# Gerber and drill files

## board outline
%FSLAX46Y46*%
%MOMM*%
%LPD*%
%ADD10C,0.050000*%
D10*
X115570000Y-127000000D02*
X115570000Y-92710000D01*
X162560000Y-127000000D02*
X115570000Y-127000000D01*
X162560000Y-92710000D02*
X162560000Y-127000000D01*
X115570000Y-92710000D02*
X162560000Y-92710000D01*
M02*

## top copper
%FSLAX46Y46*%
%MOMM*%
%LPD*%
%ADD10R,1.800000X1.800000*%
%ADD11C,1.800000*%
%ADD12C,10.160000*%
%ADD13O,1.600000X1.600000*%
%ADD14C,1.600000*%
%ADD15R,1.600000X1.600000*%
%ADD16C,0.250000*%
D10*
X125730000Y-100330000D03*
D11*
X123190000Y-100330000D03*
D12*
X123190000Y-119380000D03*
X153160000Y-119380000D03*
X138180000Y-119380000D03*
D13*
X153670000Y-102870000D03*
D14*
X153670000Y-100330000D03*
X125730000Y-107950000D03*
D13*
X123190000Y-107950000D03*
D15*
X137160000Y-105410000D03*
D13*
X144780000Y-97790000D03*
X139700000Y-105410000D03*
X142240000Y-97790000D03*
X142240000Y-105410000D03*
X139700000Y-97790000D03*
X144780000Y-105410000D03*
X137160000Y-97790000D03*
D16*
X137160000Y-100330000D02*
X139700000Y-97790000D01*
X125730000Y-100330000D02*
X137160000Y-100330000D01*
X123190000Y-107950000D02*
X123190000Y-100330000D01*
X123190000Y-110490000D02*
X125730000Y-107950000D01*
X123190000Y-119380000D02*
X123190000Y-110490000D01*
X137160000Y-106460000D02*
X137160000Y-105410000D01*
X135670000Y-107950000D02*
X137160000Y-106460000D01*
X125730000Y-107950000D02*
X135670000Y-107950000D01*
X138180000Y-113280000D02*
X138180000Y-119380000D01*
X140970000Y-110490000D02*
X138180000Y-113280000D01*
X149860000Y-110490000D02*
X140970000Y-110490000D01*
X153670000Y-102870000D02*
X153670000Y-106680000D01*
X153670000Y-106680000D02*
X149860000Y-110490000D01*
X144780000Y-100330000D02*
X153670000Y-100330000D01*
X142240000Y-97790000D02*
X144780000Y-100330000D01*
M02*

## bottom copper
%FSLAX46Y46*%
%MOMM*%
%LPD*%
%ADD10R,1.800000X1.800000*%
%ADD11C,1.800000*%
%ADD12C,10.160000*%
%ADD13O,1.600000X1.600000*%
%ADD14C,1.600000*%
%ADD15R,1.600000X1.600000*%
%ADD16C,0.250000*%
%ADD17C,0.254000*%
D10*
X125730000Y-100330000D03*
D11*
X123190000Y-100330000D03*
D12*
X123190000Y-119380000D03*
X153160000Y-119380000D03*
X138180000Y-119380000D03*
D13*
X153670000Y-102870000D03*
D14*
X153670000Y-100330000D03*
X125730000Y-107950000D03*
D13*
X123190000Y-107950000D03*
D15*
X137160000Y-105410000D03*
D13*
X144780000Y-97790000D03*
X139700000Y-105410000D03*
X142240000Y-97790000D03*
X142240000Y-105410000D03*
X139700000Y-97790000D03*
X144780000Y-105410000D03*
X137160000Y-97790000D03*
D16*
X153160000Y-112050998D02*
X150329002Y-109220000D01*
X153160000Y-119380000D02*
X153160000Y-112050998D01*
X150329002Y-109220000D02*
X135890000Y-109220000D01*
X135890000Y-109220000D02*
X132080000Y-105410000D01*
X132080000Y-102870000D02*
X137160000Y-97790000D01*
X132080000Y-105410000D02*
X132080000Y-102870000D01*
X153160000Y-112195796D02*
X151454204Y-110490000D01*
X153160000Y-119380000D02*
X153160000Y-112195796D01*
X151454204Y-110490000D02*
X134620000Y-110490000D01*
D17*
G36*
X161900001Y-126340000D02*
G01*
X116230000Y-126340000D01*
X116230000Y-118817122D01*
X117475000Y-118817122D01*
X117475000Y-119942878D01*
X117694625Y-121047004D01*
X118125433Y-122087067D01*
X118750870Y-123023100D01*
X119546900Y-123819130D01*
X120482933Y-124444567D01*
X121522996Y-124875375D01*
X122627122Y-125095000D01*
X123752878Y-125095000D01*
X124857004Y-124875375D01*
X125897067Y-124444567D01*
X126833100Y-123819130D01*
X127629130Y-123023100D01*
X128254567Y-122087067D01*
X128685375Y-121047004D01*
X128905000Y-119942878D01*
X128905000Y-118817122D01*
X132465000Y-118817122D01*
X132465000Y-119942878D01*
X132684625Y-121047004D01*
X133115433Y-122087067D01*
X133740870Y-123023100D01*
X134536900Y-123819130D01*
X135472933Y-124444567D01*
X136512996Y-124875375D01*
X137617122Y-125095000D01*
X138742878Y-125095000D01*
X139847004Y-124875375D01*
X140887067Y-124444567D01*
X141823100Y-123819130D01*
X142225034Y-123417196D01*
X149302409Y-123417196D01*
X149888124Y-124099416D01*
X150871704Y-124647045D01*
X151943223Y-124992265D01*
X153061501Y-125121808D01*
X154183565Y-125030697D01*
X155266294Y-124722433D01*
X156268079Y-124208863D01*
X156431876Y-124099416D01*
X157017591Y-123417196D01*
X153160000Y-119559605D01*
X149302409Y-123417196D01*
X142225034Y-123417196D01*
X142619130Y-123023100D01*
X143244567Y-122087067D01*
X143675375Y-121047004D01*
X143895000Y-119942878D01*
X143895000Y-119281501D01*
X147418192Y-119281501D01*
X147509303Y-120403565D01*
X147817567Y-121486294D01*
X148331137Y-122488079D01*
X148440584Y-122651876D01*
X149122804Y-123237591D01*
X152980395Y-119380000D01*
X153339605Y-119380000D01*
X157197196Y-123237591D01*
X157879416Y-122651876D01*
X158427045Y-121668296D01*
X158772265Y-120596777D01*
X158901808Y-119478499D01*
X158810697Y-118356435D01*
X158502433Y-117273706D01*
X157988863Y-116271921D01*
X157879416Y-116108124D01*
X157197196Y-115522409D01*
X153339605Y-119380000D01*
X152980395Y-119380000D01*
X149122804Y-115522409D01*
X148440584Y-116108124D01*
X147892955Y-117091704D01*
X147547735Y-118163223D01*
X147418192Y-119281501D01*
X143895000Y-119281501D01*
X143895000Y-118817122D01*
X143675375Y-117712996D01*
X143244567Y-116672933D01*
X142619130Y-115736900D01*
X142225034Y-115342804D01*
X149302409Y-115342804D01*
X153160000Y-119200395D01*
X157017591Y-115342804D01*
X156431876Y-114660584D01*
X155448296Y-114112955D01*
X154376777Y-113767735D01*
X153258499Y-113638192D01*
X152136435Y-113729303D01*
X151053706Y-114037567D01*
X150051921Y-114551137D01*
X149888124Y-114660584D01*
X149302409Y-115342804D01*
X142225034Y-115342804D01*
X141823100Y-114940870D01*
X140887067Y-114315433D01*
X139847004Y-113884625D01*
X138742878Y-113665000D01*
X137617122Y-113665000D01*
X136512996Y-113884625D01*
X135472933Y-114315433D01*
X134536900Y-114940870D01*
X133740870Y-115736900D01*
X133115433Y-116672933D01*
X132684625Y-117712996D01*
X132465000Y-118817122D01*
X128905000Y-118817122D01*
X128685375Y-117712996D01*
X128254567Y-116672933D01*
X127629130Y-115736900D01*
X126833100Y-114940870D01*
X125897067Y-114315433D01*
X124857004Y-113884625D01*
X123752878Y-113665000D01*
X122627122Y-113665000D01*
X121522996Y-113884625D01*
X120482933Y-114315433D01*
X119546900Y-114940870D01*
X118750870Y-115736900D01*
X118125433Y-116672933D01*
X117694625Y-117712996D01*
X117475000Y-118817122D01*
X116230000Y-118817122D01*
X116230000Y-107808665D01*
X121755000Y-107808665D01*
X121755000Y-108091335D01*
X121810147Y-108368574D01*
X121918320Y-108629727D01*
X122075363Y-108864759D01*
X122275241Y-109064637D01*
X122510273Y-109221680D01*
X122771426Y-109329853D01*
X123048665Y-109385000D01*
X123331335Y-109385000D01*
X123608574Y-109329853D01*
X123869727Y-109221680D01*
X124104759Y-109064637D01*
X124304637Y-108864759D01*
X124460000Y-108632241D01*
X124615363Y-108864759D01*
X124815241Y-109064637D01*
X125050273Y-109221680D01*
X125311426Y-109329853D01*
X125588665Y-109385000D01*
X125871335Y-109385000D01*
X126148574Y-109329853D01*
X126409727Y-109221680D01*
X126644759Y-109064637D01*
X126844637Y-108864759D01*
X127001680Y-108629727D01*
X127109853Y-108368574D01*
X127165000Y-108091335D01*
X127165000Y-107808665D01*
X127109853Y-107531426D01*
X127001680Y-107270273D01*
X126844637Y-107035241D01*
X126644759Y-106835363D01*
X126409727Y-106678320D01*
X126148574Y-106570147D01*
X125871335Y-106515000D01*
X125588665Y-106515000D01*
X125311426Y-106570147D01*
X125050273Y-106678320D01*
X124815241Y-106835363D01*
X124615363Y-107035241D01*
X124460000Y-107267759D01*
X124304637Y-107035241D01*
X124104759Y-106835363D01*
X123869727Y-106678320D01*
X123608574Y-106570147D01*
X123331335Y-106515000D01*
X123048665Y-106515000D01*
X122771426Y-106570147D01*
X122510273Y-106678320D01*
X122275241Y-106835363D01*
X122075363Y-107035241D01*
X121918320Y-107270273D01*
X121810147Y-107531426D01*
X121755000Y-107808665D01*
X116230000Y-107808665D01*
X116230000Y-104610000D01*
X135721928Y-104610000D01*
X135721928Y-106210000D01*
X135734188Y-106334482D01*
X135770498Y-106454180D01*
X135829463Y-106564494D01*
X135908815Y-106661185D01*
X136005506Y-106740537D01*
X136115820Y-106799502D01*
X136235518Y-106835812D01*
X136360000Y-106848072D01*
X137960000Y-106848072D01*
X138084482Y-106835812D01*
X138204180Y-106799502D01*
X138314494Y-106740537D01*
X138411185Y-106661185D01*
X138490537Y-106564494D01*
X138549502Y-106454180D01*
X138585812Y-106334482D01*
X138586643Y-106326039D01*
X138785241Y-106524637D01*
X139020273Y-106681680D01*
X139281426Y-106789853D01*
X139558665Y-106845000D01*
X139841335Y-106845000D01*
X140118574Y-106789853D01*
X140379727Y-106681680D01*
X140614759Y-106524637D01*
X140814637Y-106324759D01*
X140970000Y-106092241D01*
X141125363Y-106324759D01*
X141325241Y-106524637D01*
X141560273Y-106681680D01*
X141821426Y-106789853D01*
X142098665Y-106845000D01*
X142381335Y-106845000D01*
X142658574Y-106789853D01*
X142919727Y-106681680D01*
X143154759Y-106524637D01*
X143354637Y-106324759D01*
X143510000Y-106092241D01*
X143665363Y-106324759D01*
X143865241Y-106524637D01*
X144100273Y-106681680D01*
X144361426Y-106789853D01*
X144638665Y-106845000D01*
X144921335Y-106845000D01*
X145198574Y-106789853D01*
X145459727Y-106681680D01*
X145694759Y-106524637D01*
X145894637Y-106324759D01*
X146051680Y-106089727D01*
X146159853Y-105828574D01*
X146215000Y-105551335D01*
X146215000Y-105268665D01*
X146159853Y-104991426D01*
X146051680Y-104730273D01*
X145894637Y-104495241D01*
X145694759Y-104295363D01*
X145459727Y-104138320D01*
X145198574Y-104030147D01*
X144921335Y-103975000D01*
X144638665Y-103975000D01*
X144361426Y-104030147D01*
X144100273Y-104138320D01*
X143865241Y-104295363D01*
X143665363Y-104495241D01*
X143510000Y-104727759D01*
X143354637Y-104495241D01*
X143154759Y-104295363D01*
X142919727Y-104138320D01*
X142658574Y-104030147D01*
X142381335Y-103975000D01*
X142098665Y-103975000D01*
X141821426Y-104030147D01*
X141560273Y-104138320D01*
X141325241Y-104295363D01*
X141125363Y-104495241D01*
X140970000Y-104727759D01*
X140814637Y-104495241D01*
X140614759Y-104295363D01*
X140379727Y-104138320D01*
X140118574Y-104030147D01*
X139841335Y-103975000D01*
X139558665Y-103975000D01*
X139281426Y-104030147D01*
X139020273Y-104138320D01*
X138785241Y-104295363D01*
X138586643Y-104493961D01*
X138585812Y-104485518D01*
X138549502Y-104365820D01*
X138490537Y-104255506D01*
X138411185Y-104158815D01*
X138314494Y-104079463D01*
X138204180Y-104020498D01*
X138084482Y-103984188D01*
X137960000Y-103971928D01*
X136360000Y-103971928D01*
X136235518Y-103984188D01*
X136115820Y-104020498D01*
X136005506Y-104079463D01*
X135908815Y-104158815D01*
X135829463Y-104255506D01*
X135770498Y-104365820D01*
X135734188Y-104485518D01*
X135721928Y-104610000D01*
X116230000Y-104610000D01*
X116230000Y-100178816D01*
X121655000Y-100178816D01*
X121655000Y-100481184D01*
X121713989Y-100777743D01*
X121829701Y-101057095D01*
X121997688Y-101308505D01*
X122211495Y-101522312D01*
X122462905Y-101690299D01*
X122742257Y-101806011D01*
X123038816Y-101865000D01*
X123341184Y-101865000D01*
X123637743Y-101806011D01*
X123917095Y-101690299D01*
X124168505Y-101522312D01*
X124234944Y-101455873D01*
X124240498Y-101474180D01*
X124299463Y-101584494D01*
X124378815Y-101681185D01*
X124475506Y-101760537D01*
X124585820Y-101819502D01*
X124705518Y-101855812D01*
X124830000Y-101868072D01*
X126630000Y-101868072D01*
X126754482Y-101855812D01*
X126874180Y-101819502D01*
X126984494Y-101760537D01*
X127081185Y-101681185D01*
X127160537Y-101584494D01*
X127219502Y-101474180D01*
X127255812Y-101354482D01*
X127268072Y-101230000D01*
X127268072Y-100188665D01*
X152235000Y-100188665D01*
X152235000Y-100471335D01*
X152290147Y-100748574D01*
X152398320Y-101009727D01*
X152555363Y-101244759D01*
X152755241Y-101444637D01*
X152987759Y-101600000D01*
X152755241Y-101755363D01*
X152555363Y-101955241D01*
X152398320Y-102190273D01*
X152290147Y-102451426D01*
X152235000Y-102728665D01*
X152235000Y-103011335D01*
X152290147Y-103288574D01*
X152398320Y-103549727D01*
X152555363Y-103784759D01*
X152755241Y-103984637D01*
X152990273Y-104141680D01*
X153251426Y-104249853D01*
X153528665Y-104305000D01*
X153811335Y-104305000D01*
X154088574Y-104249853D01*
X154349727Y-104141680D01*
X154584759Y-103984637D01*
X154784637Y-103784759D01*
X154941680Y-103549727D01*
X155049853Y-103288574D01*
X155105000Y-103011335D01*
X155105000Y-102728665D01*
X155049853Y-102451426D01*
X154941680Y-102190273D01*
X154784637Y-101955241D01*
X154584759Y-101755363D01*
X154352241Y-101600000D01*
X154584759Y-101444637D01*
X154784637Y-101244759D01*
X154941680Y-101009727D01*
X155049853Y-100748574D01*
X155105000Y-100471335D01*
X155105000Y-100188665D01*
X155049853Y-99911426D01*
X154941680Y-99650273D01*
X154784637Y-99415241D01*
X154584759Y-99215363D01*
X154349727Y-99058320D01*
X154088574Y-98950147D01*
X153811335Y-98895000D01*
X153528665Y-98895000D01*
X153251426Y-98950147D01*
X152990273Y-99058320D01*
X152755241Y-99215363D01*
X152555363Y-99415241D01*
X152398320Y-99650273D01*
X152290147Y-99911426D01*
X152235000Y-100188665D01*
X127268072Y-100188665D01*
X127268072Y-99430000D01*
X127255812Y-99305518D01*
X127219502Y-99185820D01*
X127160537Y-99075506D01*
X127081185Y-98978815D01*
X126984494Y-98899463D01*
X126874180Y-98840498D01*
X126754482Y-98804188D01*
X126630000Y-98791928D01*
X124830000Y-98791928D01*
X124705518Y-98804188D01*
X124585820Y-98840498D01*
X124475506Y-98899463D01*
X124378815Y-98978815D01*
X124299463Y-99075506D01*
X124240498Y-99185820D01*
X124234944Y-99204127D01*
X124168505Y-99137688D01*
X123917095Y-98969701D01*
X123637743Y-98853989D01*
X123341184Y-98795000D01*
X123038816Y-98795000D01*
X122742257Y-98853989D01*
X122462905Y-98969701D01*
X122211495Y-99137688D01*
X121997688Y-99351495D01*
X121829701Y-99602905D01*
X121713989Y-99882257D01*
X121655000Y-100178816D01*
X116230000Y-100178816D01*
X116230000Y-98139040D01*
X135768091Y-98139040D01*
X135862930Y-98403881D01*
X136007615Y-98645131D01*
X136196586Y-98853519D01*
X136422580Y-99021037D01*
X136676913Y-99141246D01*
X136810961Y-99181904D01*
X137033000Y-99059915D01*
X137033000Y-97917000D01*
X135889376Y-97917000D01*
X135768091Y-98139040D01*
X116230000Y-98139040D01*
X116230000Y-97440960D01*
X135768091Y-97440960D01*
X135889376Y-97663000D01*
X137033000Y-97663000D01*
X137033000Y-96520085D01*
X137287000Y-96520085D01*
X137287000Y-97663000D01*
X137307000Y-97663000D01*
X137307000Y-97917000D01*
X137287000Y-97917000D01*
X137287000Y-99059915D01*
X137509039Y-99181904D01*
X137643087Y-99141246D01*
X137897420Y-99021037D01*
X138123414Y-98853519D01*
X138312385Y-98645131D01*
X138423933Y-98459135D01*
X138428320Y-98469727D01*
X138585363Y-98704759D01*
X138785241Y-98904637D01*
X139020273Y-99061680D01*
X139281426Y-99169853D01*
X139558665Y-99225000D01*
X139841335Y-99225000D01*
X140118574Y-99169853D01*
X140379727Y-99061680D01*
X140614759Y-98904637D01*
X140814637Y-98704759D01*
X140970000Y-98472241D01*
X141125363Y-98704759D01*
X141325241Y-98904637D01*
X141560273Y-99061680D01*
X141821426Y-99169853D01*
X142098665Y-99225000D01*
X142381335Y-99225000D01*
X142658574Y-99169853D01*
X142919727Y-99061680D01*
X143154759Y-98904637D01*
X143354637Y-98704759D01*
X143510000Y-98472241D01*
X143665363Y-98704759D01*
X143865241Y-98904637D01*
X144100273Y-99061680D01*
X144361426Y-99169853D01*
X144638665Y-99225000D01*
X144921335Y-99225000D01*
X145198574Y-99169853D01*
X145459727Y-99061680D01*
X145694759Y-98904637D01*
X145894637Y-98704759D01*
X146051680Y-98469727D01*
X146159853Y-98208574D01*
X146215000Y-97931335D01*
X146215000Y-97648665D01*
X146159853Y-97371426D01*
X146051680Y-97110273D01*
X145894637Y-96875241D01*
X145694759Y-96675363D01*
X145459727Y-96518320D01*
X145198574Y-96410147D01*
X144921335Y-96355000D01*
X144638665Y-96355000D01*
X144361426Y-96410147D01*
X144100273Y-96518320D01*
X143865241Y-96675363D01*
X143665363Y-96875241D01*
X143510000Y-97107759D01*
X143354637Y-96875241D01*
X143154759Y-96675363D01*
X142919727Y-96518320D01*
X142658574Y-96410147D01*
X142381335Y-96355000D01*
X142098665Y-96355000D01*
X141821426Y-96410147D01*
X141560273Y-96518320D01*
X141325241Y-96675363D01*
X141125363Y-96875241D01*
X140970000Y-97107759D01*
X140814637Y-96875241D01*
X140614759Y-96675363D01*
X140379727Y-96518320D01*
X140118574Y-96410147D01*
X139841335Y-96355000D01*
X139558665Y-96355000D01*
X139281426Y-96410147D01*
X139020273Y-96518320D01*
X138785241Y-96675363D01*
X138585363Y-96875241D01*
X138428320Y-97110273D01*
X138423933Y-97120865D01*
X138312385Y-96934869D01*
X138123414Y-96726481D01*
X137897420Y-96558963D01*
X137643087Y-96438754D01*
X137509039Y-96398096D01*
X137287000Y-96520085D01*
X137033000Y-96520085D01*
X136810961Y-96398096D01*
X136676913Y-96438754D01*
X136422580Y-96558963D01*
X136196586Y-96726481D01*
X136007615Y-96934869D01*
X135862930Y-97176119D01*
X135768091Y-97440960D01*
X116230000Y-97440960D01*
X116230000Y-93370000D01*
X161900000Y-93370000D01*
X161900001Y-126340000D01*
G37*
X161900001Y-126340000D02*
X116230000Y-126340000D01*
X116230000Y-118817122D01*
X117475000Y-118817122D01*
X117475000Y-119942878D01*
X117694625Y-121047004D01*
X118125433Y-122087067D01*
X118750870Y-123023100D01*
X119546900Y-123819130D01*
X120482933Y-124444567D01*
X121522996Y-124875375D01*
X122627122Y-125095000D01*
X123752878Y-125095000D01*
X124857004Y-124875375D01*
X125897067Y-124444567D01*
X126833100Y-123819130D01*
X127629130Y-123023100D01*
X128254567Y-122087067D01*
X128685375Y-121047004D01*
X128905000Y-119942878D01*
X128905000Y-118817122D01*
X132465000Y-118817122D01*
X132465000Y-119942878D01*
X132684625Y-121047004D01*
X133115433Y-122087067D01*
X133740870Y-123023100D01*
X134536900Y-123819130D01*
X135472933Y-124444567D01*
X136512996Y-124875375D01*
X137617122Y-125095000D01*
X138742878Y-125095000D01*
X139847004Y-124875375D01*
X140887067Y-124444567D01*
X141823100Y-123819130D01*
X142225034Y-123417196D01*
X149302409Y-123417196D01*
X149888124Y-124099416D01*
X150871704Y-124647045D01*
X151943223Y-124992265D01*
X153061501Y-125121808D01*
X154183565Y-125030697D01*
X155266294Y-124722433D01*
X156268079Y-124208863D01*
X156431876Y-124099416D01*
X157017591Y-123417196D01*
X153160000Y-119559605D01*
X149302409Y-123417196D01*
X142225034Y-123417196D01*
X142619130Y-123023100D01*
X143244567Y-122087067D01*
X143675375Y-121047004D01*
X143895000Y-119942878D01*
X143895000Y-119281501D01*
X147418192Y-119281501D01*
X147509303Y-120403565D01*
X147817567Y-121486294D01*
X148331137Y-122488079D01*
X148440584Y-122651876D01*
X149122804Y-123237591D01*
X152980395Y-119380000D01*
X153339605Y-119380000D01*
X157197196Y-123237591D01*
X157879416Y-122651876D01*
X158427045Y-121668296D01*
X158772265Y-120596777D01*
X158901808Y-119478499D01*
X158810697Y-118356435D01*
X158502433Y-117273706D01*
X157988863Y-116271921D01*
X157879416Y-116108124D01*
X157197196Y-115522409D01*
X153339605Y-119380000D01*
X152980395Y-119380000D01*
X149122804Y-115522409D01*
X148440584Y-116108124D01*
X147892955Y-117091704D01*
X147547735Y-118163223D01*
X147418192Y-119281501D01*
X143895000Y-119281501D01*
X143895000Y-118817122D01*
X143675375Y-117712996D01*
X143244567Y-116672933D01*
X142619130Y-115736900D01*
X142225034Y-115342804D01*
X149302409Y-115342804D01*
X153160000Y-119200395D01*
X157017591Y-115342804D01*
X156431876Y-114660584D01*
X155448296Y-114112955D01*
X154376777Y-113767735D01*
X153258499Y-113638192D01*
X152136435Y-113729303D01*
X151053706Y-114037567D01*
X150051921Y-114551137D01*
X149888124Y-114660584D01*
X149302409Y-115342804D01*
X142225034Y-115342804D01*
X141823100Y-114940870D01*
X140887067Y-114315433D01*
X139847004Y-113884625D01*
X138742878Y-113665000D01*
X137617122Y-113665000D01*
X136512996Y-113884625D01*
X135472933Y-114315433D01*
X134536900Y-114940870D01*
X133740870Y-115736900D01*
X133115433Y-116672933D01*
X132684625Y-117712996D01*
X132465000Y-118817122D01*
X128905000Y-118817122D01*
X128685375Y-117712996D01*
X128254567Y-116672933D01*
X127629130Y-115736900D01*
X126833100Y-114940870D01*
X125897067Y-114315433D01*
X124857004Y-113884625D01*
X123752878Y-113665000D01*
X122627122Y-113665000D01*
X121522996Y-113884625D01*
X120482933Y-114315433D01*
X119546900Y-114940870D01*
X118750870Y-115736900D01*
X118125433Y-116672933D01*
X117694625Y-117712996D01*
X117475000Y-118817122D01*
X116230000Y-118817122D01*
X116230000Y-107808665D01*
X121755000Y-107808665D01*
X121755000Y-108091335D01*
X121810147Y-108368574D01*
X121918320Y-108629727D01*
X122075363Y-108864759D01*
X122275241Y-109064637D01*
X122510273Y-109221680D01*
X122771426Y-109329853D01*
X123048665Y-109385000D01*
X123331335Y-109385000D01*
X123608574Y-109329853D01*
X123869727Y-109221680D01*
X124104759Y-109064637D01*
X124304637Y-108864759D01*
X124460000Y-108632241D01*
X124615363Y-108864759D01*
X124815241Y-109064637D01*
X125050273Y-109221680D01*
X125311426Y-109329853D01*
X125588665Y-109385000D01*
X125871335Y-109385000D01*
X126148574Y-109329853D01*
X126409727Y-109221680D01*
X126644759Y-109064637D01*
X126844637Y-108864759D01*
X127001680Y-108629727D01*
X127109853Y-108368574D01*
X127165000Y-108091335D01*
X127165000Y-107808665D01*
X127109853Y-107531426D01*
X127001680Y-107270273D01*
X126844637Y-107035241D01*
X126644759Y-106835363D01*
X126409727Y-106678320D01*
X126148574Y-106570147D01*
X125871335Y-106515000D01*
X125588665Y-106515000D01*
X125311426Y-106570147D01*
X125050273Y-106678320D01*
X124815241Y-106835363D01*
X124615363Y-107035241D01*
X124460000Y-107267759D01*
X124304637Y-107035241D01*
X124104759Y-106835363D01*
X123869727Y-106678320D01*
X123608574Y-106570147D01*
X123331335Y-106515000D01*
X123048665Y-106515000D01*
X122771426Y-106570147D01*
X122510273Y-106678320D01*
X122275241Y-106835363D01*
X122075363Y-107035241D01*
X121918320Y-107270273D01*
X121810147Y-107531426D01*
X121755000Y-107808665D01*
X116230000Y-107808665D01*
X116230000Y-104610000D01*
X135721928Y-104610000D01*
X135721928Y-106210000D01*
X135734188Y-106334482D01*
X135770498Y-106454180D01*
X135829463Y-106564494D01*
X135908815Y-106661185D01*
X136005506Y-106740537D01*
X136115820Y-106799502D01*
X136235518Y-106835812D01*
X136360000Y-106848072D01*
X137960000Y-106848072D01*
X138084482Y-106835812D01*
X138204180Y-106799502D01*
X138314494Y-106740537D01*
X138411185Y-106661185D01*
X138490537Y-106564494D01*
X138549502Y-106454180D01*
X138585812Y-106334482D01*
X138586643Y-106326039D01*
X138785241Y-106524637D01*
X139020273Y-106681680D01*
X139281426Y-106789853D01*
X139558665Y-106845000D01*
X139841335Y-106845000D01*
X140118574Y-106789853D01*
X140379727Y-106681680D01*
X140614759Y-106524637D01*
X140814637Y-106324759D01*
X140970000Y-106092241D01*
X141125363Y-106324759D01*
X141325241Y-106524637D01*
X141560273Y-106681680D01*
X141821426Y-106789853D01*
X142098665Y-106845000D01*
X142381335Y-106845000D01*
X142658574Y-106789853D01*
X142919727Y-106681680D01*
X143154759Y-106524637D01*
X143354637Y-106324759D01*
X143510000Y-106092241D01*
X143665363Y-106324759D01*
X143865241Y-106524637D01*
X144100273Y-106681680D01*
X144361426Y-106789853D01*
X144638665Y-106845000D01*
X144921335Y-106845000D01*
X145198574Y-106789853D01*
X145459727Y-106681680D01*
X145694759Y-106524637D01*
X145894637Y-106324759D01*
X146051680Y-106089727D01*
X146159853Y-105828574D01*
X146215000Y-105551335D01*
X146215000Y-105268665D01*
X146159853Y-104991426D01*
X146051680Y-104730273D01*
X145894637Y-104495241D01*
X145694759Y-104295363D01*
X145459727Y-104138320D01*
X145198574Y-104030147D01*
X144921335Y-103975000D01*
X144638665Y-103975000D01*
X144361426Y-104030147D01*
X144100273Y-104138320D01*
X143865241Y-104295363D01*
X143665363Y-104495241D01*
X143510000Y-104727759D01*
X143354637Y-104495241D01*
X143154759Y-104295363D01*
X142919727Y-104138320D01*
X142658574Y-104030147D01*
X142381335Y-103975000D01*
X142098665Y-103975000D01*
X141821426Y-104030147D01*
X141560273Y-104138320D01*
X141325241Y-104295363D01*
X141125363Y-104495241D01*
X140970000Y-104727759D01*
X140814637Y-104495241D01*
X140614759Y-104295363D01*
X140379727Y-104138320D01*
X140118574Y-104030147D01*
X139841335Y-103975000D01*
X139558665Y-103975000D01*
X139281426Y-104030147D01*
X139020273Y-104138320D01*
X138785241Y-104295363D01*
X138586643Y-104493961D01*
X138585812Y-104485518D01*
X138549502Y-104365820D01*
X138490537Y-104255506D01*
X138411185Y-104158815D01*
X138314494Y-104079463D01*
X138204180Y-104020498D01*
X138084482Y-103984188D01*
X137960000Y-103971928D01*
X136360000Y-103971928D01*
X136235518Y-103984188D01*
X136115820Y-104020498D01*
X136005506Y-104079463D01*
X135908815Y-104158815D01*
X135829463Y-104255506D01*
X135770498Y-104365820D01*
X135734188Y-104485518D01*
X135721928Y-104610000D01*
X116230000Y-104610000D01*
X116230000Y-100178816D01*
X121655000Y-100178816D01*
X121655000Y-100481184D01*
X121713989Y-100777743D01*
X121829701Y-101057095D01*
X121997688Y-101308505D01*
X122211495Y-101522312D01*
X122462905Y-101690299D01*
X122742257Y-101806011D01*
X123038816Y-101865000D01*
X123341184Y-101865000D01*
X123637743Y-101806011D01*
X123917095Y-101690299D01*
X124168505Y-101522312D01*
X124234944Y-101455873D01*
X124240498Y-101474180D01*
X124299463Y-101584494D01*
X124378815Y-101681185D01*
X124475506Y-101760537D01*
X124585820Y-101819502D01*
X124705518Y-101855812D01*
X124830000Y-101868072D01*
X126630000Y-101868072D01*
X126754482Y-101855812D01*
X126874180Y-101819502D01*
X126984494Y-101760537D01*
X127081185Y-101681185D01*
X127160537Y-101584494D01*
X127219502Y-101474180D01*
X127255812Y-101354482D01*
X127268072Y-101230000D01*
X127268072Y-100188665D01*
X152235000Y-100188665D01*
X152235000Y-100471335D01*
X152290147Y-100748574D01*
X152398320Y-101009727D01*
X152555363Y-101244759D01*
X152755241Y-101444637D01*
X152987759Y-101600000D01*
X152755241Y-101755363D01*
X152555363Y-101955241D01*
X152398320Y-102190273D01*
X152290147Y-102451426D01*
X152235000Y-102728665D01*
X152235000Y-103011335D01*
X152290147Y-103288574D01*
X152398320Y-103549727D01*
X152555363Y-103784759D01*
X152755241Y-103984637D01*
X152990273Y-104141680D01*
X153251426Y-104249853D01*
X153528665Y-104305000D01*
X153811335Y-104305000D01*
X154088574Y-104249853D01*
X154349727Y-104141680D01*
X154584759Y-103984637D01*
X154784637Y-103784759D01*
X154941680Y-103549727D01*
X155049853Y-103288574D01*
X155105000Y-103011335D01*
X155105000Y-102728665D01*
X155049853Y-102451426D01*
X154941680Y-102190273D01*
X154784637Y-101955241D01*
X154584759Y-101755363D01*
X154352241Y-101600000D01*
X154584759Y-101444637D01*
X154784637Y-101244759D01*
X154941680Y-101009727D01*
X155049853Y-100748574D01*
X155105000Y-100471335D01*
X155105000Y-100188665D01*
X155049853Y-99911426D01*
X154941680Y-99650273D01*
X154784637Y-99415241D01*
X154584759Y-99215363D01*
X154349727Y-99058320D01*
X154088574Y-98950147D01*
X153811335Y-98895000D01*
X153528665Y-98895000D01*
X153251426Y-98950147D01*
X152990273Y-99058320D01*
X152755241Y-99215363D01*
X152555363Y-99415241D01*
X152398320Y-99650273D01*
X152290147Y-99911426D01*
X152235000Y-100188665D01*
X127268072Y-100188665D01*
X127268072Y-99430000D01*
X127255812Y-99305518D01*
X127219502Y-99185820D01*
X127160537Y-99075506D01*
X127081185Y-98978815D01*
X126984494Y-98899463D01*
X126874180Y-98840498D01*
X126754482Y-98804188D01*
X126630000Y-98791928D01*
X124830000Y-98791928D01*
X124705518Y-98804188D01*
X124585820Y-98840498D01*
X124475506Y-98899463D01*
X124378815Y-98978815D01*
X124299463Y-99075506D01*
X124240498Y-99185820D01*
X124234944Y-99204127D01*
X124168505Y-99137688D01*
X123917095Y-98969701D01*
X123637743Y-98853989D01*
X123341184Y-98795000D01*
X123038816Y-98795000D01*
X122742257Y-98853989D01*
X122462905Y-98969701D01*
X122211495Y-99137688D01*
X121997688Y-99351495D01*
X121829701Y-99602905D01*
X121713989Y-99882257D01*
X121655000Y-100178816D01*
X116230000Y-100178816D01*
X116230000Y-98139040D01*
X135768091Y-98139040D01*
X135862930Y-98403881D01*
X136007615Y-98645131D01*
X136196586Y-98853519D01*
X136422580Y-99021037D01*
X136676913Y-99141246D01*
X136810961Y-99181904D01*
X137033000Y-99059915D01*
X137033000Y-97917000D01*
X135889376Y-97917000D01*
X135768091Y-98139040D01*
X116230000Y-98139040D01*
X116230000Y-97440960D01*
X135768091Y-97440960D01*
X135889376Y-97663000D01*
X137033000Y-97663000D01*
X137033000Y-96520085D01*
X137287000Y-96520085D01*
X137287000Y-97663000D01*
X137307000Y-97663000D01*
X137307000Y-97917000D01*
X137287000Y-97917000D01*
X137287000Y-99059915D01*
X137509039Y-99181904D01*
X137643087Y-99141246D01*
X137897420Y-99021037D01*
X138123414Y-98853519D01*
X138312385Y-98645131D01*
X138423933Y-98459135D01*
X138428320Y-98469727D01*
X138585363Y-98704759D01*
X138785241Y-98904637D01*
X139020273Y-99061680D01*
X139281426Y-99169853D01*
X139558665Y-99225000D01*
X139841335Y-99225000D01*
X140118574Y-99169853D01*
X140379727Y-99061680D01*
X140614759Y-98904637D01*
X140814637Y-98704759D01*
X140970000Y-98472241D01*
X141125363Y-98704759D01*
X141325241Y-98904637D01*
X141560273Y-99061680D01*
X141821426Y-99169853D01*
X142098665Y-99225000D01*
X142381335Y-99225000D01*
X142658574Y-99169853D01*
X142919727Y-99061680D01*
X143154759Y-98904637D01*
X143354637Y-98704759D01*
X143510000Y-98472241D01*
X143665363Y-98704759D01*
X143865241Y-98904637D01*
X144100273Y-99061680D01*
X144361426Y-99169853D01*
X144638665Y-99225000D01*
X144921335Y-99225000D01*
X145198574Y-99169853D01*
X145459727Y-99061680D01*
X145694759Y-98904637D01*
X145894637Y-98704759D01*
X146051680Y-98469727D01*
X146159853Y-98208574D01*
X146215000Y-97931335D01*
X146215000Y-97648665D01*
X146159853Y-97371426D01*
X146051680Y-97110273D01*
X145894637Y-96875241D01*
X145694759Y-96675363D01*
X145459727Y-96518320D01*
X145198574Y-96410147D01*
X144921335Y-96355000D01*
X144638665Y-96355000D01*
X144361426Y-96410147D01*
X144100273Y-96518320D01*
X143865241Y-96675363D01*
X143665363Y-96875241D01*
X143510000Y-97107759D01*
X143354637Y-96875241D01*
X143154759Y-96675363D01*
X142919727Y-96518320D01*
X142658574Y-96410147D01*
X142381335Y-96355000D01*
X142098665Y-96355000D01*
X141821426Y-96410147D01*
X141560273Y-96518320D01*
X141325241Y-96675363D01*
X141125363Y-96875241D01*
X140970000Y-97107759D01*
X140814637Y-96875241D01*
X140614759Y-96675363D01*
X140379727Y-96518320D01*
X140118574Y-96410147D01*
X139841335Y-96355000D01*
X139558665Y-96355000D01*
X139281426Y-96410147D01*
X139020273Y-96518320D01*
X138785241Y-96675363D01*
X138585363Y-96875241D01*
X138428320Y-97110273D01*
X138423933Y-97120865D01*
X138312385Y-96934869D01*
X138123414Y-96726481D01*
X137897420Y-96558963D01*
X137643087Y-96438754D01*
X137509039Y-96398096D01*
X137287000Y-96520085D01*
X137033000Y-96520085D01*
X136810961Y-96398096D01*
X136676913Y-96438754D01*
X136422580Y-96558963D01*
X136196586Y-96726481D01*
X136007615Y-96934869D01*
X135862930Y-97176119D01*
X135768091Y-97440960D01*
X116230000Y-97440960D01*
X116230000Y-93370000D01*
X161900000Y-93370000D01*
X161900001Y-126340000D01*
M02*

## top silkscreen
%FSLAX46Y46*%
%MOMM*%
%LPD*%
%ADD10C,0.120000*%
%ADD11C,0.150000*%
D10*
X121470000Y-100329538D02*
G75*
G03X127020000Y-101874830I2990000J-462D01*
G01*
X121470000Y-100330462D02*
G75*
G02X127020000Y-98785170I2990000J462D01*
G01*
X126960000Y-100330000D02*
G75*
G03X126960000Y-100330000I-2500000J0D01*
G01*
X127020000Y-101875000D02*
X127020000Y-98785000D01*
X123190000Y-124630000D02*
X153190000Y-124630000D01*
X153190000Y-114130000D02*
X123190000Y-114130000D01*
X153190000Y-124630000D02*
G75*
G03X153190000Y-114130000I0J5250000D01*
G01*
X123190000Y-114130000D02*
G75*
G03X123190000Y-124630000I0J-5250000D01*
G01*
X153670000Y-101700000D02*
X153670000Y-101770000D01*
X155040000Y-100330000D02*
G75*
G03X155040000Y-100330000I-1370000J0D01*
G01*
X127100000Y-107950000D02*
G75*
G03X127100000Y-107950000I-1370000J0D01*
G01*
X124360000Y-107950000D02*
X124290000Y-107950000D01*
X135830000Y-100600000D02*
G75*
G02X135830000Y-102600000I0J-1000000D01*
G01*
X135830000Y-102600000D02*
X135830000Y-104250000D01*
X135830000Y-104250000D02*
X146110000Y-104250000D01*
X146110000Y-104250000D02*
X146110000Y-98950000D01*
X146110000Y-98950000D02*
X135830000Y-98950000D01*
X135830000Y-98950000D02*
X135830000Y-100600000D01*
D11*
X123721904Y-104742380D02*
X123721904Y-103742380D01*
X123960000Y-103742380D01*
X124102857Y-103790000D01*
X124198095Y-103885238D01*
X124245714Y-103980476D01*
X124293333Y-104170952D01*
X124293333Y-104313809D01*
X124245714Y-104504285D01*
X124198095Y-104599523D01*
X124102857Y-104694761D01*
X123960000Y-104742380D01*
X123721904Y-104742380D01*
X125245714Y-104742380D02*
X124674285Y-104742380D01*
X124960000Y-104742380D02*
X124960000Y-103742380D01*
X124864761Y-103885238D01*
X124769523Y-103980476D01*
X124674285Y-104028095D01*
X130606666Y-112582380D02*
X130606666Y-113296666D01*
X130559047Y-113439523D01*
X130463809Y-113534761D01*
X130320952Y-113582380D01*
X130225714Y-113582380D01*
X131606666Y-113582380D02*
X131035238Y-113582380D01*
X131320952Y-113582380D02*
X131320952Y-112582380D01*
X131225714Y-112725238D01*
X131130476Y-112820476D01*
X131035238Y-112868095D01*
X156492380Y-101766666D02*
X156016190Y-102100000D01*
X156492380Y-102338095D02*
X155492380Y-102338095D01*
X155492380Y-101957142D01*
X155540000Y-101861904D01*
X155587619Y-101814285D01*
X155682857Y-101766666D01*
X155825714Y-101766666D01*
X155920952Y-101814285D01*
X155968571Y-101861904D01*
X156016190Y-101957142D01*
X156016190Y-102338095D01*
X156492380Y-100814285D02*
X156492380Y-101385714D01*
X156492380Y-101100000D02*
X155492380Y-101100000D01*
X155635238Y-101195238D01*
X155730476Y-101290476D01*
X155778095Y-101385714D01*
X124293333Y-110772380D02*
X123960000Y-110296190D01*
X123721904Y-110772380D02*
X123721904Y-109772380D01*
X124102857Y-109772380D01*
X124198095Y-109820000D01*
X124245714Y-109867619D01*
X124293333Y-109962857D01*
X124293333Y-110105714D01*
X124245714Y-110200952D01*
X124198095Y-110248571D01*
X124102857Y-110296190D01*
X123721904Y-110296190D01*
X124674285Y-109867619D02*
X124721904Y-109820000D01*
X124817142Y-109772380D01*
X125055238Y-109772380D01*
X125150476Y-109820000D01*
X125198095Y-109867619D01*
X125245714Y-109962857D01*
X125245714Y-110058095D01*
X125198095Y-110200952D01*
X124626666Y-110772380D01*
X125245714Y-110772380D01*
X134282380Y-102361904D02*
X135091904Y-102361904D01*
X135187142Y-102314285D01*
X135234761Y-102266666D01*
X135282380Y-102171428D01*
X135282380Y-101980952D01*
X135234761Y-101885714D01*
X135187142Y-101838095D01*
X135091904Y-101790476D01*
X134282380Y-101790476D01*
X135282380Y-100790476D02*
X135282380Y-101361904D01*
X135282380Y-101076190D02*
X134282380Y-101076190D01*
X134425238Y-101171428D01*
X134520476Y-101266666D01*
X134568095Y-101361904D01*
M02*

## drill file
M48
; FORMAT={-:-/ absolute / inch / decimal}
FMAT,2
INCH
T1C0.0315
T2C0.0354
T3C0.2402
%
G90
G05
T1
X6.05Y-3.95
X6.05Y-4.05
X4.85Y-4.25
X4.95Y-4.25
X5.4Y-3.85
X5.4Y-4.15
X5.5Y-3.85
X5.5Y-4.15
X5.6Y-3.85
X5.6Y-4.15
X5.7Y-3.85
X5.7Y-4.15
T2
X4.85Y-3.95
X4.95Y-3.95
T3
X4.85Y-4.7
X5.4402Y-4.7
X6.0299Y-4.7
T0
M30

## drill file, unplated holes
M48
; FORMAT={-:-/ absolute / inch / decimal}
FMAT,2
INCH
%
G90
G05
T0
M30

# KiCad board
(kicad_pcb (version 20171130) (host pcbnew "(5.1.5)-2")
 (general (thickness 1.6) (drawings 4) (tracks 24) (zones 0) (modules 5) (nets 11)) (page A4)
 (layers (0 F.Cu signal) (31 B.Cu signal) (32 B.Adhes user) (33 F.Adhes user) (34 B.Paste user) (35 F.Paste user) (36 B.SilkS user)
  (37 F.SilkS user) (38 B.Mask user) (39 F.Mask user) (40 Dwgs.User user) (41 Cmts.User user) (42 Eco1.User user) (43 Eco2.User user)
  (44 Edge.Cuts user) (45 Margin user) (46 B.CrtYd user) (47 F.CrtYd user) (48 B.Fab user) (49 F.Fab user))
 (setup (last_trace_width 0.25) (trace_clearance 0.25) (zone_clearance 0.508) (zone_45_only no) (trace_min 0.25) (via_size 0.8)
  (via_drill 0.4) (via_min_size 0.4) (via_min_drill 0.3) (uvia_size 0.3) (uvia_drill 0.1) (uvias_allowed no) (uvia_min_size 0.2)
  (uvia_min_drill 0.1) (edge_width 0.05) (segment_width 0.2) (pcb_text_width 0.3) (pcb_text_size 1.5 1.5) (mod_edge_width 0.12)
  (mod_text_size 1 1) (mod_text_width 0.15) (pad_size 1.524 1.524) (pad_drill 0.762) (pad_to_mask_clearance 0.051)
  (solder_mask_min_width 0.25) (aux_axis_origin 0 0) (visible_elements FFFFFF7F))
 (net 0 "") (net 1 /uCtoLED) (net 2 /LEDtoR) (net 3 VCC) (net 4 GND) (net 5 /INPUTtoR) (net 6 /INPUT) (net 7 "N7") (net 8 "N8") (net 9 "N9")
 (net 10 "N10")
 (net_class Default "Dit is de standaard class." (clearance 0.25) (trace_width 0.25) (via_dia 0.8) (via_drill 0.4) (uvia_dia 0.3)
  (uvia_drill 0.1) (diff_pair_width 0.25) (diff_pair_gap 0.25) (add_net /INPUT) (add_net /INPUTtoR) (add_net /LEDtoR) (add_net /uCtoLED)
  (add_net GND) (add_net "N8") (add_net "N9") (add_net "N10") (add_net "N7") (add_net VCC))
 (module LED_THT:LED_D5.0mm (layer F.Cu) (at 125.73 100.33 180)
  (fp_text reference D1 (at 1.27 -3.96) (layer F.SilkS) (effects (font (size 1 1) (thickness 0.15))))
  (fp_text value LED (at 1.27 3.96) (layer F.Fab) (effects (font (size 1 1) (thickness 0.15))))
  (fp_arc (start 1.27 0) (end -1.29 -1.54483) (angle 148.9) (layer F.SilkS) (width 0.12))
  (fp_arc (start 1.27 0) (end -1.29 1.54483) (angle -148.9) (layer F.SilkS) (width 0.12))
  (fp_circle (center 1.27 0) (end 3.77 0) (layer F.SilkS) (width 0.12))
  (fp_line (start -1.29 -1.545) (end -1.29 1.545) (layer F.SilkS) (width 0.12))
  (pad 1 thru_hole rect (at 0 0 180) (size 1.8 1.8) (drill 0.9) (layers *.Cu *.Mask) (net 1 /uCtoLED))
  (pad 2 thru_hole circle (at 2.54 0 180) (size 1.8 1.8) (drill 0.9) (layers *.Cu *.Mask) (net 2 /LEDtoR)))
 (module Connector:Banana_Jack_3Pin (layer F.Cu) (at 123.19 119.38)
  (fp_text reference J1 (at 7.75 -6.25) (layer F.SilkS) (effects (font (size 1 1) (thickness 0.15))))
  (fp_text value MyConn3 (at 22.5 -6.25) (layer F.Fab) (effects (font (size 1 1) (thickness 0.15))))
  (fp_line (start 0 5.25) (end 30 5.25) (layer F.SilkS) (width 0.12))
  (fp_line (start 30 -5.25) (end 0 -5.25) (layer F.SilkS) (width 0.12))
  (fp_arc (start 30 0) (end 30 -5.25) (angle 180) (layer F.SilkS) (width 0.12))
  (fp_arc (start 0 0) (end 0 5.25) (angle 180) (layer F.SilkS) (width 0.12))
  (pad 1 thru_hole circle (at 0 0) (size 10.16 10.16) (drill 6.1) (layers *.Cu *.Mask) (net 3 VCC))
  (pad 3 thru_hole circle (at 29.97 0) (size 10.16 10.16) (drill 6.1) (layers *.Cu *.Mask) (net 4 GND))
  (pad 2 thru_hole circle (at 14.99 0) (size 10.16 10.16) (drill 6.1) (layers *.Cu *.Mask) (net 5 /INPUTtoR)))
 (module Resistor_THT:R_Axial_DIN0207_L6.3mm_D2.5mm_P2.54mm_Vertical (layer F.Cu) (at 153.67 100.33 270)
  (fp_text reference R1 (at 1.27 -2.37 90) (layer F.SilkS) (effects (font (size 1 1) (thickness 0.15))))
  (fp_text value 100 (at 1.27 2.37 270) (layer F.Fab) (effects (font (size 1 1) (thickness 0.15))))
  (fp_line (start 1.37 0) (end 1.44 0) (layer F.SilkS) (width 0.12))
  (fp_circle (center 0 0) (end 1.37 0) (layer F.SilkS) (width 0.12))
  (pad 2 thru_hole oval (at 2.54 0 270) (size 1.6 1.6) (drill 0.8) (layers *.Cu *.Mask) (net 5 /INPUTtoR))
  (pad 1 thru_hole circle (at 0 0 270) (size 1.6 1.6) (drill 0.8) (layers *.Cu *.Mask) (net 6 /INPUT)))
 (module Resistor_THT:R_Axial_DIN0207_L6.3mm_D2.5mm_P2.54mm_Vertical (layer F.Cu) (at 125.73 107.95 180)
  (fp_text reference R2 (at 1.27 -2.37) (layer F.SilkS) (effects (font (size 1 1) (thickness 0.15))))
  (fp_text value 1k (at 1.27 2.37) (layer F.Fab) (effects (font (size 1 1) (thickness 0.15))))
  (fp_circle (center 0 0) (end 1.37 0) (layer F.SilkS) (width 0.12))
  (fp_line (start 1.37 0) (end 1.44 0) (layer F.SilkS) (width 0.12))
  (pad 1 thru_hole circle (at 0 0 180) (size 1.6 1.6) (drill 0.8) (layers *.Cu *.Mask) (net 3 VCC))
  (pad 2 thru_hole oval (at 2.54 0 180) (size 1.6 1.6) (drill 0.8) (layers *.Cu *.Mask) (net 2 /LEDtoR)))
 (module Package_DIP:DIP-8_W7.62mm (layer F.Cu) (at 137.16 105.41 90)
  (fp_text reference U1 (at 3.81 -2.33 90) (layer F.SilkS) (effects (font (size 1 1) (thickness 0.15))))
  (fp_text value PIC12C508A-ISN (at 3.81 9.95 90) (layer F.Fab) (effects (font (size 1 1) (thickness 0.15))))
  (fp_arc (start 3.81 -1.33) (end 2.81 -1.33) (angle -180) (layer F.SilkS) (width 0.12))
  (fp_line (start 2.81 -1.33) (end 1.16 -1.33) (layer F.SilkS) (width 0.12))
  (fp_line (start 1.16 -1.33) (end 1.16 8.95) (layer F.SilkS) (width 0.12))
  (fp_line (start 1.16 8.95) (end 6.46 8.95) (layer F.SilkS) (width 0.12))
  (fp_line (start 6.46 8.95) (end 6.46 -1.33) (layer F.SilkS) (width 0.12))
  (fp_line (start 6.46 -1.33) (end 4.81 -1.33) (layer F.SilkS) (width 0.12))
  (pad 1 thru_hole rect (at 0 0 90) (size 1.6 1.6) (drill 0.8) (layers *.Cu *.Mask) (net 3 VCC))
  (pad 5 thru_hole oval (at 7.62 7.62 90) (size 1.6 1.6) (drill 0.8) (layers *.Cu *.Mask) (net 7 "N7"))
  (pad 2 thru_hole oval (at 0 2.54 90) (size 1.6 1.6) (drill 0.8) (layers *.Cu *.Mask) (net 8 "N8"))
  (pad 6 thru_hole oval (at 7.62 5.08 90) (size 1.6 1.6) (drill 0.8) (layers *.Cu *.Mask) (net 6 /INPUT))
  (pad 3 thru_hole oval (at 0 5.08 90) (size 1.6 1.6) (drill 0.8) (layers *.Cu *.Mask) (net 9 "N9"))
  (pad 7 thru_hole oval (at 7.62 2.54 90) (size 1.6 1.6) (drill 0.8) (layers *.Cu *.Mask) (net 1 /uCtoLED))
  (pad 4 thru_hole oval (at 0 7.62 90) (size 1.6 1.6) (drill 0.8) (layers *.Cu *.Mask) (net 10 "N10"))
  (pad 8 thru_hole oval (at 7.62 0 90) (size 1.6 1.6) (drill 0.8) (layers *.Cu *.Mask) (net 4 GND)))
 (gr_line (start 115.57 127) (end 115.57 92.71) (layer Edge.Cuts) (width 0.05))
 (gr_line (start 162.56 127) (end 115.57 127) (layer Edge.Cuts) (width 0.05))
 (gr_line (start 162.56 92.71) (end 162.56 127) (layer Edge.Cuts) (width 0.05))
 (gr_line (start 115.57 92.71) (end 162.56 92.71) (layer Edge.Cuts) (width 0.05))
 (segment (start 137.16 100.33) (end 139.7 97.79) (width 0.25) (layer F.Cu) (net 1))
 (segment (start 125.73 100.33) (end 137.16 100.33) (width 0.25) (layer F.Cu) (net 1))
 (segment (start 123.19 107.95) (end 123.19 100.33) (width 0.25) (layer F.Cu) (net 2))
 (segment (start 123.19 110.49) (end 125.73 107.95) (width 0.25) (layer F.Cu) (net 3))
 (segment (start 123.19 119.38) (end 123.19 110.49) (width 0.25) (layer F.Cu) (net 3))
 (segment (start 137.16 106.46) (end 137.16 105.41) (width 0.25) (layer F.Cu) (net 3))
 (segment (start 135.67 107.95) (end 137.16 106.46) (width 0.25) (layer F.Cu) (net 3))
 (segment (start 125.73 107.95) (end 135.67 107.95) (width 0.25) (layer F.Cu) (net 3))
 (segment (start 153.16 112.050998) (end 150.329002 109.22) (width 0.25) (layer B.Cu) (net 4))
 (segment (start 153.16 119.38) (end 153.16 112.050998) (width 0.25) (layer B.Cu) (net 4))
 (segment (start 150.329002 109.22) (end 135.89 109.22) (width 0.25) (layer B.Cu) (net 4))
 (segment (start 135.89 109.22) (end 132.08 105.41) (width 0.25) (layer B.Cu) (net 4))
 (segment (start 132.08 102.87) (end 137.16 97.79) (width 0.25) (layer B.Cu) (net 4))
 (segment (start 132.08 105.41) (end 132.08 102.87) (width 0.25) (layer B.Cu) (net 4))
 (segment (start 153.16 112.195796) (end 151.454204 110.49) (width 0.25) (layer B.Cu) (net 4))
 (segment (start 153.16 119.38) (end 153.16 112.195796) (width 0.25) (layer B.Cu) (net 4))
 (segment (start 151.454204 110.49) (end 134.62 110.49) (width 0.25) (layer B.Cu) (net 4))
 (segment (start 138.18 113.28) (end 138.18 119.38) (width 0.25) (layer F.Cu) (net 5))
 (segment (start 140.97 110.49) (end 138.18 113.28) (width 0.25) (layer F.Cu) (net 5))
 (segment (start 149.86 110.49) (end 140.97 110.49) (width 0.25) (layer F.Cu) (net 5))
 (segment (start 153.67 102.87) (end 153.67 106.68) (width 0.25) (layer F.Cu) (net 5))
 (segment (start 153.67 106.68) (end 149.86 110.49) (width 0.25) (layer F.Cu) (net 5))
 (segment (start 144.78 100.33) (end 153.67 100.33) (width 0.25) (layer F.Cu) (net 6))
 (segment (start 142.24 97.79) (end 144.78 100.33) (width 0.25) (layer F.Cu) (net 6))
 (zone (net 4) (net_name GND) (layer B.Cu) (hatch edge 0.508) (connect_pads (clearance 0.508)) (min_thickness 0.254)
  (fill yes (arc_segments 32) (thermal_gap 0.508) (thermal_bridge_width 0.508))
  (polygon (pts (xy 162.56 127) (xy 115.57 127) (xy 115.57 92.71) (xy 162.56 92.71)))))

